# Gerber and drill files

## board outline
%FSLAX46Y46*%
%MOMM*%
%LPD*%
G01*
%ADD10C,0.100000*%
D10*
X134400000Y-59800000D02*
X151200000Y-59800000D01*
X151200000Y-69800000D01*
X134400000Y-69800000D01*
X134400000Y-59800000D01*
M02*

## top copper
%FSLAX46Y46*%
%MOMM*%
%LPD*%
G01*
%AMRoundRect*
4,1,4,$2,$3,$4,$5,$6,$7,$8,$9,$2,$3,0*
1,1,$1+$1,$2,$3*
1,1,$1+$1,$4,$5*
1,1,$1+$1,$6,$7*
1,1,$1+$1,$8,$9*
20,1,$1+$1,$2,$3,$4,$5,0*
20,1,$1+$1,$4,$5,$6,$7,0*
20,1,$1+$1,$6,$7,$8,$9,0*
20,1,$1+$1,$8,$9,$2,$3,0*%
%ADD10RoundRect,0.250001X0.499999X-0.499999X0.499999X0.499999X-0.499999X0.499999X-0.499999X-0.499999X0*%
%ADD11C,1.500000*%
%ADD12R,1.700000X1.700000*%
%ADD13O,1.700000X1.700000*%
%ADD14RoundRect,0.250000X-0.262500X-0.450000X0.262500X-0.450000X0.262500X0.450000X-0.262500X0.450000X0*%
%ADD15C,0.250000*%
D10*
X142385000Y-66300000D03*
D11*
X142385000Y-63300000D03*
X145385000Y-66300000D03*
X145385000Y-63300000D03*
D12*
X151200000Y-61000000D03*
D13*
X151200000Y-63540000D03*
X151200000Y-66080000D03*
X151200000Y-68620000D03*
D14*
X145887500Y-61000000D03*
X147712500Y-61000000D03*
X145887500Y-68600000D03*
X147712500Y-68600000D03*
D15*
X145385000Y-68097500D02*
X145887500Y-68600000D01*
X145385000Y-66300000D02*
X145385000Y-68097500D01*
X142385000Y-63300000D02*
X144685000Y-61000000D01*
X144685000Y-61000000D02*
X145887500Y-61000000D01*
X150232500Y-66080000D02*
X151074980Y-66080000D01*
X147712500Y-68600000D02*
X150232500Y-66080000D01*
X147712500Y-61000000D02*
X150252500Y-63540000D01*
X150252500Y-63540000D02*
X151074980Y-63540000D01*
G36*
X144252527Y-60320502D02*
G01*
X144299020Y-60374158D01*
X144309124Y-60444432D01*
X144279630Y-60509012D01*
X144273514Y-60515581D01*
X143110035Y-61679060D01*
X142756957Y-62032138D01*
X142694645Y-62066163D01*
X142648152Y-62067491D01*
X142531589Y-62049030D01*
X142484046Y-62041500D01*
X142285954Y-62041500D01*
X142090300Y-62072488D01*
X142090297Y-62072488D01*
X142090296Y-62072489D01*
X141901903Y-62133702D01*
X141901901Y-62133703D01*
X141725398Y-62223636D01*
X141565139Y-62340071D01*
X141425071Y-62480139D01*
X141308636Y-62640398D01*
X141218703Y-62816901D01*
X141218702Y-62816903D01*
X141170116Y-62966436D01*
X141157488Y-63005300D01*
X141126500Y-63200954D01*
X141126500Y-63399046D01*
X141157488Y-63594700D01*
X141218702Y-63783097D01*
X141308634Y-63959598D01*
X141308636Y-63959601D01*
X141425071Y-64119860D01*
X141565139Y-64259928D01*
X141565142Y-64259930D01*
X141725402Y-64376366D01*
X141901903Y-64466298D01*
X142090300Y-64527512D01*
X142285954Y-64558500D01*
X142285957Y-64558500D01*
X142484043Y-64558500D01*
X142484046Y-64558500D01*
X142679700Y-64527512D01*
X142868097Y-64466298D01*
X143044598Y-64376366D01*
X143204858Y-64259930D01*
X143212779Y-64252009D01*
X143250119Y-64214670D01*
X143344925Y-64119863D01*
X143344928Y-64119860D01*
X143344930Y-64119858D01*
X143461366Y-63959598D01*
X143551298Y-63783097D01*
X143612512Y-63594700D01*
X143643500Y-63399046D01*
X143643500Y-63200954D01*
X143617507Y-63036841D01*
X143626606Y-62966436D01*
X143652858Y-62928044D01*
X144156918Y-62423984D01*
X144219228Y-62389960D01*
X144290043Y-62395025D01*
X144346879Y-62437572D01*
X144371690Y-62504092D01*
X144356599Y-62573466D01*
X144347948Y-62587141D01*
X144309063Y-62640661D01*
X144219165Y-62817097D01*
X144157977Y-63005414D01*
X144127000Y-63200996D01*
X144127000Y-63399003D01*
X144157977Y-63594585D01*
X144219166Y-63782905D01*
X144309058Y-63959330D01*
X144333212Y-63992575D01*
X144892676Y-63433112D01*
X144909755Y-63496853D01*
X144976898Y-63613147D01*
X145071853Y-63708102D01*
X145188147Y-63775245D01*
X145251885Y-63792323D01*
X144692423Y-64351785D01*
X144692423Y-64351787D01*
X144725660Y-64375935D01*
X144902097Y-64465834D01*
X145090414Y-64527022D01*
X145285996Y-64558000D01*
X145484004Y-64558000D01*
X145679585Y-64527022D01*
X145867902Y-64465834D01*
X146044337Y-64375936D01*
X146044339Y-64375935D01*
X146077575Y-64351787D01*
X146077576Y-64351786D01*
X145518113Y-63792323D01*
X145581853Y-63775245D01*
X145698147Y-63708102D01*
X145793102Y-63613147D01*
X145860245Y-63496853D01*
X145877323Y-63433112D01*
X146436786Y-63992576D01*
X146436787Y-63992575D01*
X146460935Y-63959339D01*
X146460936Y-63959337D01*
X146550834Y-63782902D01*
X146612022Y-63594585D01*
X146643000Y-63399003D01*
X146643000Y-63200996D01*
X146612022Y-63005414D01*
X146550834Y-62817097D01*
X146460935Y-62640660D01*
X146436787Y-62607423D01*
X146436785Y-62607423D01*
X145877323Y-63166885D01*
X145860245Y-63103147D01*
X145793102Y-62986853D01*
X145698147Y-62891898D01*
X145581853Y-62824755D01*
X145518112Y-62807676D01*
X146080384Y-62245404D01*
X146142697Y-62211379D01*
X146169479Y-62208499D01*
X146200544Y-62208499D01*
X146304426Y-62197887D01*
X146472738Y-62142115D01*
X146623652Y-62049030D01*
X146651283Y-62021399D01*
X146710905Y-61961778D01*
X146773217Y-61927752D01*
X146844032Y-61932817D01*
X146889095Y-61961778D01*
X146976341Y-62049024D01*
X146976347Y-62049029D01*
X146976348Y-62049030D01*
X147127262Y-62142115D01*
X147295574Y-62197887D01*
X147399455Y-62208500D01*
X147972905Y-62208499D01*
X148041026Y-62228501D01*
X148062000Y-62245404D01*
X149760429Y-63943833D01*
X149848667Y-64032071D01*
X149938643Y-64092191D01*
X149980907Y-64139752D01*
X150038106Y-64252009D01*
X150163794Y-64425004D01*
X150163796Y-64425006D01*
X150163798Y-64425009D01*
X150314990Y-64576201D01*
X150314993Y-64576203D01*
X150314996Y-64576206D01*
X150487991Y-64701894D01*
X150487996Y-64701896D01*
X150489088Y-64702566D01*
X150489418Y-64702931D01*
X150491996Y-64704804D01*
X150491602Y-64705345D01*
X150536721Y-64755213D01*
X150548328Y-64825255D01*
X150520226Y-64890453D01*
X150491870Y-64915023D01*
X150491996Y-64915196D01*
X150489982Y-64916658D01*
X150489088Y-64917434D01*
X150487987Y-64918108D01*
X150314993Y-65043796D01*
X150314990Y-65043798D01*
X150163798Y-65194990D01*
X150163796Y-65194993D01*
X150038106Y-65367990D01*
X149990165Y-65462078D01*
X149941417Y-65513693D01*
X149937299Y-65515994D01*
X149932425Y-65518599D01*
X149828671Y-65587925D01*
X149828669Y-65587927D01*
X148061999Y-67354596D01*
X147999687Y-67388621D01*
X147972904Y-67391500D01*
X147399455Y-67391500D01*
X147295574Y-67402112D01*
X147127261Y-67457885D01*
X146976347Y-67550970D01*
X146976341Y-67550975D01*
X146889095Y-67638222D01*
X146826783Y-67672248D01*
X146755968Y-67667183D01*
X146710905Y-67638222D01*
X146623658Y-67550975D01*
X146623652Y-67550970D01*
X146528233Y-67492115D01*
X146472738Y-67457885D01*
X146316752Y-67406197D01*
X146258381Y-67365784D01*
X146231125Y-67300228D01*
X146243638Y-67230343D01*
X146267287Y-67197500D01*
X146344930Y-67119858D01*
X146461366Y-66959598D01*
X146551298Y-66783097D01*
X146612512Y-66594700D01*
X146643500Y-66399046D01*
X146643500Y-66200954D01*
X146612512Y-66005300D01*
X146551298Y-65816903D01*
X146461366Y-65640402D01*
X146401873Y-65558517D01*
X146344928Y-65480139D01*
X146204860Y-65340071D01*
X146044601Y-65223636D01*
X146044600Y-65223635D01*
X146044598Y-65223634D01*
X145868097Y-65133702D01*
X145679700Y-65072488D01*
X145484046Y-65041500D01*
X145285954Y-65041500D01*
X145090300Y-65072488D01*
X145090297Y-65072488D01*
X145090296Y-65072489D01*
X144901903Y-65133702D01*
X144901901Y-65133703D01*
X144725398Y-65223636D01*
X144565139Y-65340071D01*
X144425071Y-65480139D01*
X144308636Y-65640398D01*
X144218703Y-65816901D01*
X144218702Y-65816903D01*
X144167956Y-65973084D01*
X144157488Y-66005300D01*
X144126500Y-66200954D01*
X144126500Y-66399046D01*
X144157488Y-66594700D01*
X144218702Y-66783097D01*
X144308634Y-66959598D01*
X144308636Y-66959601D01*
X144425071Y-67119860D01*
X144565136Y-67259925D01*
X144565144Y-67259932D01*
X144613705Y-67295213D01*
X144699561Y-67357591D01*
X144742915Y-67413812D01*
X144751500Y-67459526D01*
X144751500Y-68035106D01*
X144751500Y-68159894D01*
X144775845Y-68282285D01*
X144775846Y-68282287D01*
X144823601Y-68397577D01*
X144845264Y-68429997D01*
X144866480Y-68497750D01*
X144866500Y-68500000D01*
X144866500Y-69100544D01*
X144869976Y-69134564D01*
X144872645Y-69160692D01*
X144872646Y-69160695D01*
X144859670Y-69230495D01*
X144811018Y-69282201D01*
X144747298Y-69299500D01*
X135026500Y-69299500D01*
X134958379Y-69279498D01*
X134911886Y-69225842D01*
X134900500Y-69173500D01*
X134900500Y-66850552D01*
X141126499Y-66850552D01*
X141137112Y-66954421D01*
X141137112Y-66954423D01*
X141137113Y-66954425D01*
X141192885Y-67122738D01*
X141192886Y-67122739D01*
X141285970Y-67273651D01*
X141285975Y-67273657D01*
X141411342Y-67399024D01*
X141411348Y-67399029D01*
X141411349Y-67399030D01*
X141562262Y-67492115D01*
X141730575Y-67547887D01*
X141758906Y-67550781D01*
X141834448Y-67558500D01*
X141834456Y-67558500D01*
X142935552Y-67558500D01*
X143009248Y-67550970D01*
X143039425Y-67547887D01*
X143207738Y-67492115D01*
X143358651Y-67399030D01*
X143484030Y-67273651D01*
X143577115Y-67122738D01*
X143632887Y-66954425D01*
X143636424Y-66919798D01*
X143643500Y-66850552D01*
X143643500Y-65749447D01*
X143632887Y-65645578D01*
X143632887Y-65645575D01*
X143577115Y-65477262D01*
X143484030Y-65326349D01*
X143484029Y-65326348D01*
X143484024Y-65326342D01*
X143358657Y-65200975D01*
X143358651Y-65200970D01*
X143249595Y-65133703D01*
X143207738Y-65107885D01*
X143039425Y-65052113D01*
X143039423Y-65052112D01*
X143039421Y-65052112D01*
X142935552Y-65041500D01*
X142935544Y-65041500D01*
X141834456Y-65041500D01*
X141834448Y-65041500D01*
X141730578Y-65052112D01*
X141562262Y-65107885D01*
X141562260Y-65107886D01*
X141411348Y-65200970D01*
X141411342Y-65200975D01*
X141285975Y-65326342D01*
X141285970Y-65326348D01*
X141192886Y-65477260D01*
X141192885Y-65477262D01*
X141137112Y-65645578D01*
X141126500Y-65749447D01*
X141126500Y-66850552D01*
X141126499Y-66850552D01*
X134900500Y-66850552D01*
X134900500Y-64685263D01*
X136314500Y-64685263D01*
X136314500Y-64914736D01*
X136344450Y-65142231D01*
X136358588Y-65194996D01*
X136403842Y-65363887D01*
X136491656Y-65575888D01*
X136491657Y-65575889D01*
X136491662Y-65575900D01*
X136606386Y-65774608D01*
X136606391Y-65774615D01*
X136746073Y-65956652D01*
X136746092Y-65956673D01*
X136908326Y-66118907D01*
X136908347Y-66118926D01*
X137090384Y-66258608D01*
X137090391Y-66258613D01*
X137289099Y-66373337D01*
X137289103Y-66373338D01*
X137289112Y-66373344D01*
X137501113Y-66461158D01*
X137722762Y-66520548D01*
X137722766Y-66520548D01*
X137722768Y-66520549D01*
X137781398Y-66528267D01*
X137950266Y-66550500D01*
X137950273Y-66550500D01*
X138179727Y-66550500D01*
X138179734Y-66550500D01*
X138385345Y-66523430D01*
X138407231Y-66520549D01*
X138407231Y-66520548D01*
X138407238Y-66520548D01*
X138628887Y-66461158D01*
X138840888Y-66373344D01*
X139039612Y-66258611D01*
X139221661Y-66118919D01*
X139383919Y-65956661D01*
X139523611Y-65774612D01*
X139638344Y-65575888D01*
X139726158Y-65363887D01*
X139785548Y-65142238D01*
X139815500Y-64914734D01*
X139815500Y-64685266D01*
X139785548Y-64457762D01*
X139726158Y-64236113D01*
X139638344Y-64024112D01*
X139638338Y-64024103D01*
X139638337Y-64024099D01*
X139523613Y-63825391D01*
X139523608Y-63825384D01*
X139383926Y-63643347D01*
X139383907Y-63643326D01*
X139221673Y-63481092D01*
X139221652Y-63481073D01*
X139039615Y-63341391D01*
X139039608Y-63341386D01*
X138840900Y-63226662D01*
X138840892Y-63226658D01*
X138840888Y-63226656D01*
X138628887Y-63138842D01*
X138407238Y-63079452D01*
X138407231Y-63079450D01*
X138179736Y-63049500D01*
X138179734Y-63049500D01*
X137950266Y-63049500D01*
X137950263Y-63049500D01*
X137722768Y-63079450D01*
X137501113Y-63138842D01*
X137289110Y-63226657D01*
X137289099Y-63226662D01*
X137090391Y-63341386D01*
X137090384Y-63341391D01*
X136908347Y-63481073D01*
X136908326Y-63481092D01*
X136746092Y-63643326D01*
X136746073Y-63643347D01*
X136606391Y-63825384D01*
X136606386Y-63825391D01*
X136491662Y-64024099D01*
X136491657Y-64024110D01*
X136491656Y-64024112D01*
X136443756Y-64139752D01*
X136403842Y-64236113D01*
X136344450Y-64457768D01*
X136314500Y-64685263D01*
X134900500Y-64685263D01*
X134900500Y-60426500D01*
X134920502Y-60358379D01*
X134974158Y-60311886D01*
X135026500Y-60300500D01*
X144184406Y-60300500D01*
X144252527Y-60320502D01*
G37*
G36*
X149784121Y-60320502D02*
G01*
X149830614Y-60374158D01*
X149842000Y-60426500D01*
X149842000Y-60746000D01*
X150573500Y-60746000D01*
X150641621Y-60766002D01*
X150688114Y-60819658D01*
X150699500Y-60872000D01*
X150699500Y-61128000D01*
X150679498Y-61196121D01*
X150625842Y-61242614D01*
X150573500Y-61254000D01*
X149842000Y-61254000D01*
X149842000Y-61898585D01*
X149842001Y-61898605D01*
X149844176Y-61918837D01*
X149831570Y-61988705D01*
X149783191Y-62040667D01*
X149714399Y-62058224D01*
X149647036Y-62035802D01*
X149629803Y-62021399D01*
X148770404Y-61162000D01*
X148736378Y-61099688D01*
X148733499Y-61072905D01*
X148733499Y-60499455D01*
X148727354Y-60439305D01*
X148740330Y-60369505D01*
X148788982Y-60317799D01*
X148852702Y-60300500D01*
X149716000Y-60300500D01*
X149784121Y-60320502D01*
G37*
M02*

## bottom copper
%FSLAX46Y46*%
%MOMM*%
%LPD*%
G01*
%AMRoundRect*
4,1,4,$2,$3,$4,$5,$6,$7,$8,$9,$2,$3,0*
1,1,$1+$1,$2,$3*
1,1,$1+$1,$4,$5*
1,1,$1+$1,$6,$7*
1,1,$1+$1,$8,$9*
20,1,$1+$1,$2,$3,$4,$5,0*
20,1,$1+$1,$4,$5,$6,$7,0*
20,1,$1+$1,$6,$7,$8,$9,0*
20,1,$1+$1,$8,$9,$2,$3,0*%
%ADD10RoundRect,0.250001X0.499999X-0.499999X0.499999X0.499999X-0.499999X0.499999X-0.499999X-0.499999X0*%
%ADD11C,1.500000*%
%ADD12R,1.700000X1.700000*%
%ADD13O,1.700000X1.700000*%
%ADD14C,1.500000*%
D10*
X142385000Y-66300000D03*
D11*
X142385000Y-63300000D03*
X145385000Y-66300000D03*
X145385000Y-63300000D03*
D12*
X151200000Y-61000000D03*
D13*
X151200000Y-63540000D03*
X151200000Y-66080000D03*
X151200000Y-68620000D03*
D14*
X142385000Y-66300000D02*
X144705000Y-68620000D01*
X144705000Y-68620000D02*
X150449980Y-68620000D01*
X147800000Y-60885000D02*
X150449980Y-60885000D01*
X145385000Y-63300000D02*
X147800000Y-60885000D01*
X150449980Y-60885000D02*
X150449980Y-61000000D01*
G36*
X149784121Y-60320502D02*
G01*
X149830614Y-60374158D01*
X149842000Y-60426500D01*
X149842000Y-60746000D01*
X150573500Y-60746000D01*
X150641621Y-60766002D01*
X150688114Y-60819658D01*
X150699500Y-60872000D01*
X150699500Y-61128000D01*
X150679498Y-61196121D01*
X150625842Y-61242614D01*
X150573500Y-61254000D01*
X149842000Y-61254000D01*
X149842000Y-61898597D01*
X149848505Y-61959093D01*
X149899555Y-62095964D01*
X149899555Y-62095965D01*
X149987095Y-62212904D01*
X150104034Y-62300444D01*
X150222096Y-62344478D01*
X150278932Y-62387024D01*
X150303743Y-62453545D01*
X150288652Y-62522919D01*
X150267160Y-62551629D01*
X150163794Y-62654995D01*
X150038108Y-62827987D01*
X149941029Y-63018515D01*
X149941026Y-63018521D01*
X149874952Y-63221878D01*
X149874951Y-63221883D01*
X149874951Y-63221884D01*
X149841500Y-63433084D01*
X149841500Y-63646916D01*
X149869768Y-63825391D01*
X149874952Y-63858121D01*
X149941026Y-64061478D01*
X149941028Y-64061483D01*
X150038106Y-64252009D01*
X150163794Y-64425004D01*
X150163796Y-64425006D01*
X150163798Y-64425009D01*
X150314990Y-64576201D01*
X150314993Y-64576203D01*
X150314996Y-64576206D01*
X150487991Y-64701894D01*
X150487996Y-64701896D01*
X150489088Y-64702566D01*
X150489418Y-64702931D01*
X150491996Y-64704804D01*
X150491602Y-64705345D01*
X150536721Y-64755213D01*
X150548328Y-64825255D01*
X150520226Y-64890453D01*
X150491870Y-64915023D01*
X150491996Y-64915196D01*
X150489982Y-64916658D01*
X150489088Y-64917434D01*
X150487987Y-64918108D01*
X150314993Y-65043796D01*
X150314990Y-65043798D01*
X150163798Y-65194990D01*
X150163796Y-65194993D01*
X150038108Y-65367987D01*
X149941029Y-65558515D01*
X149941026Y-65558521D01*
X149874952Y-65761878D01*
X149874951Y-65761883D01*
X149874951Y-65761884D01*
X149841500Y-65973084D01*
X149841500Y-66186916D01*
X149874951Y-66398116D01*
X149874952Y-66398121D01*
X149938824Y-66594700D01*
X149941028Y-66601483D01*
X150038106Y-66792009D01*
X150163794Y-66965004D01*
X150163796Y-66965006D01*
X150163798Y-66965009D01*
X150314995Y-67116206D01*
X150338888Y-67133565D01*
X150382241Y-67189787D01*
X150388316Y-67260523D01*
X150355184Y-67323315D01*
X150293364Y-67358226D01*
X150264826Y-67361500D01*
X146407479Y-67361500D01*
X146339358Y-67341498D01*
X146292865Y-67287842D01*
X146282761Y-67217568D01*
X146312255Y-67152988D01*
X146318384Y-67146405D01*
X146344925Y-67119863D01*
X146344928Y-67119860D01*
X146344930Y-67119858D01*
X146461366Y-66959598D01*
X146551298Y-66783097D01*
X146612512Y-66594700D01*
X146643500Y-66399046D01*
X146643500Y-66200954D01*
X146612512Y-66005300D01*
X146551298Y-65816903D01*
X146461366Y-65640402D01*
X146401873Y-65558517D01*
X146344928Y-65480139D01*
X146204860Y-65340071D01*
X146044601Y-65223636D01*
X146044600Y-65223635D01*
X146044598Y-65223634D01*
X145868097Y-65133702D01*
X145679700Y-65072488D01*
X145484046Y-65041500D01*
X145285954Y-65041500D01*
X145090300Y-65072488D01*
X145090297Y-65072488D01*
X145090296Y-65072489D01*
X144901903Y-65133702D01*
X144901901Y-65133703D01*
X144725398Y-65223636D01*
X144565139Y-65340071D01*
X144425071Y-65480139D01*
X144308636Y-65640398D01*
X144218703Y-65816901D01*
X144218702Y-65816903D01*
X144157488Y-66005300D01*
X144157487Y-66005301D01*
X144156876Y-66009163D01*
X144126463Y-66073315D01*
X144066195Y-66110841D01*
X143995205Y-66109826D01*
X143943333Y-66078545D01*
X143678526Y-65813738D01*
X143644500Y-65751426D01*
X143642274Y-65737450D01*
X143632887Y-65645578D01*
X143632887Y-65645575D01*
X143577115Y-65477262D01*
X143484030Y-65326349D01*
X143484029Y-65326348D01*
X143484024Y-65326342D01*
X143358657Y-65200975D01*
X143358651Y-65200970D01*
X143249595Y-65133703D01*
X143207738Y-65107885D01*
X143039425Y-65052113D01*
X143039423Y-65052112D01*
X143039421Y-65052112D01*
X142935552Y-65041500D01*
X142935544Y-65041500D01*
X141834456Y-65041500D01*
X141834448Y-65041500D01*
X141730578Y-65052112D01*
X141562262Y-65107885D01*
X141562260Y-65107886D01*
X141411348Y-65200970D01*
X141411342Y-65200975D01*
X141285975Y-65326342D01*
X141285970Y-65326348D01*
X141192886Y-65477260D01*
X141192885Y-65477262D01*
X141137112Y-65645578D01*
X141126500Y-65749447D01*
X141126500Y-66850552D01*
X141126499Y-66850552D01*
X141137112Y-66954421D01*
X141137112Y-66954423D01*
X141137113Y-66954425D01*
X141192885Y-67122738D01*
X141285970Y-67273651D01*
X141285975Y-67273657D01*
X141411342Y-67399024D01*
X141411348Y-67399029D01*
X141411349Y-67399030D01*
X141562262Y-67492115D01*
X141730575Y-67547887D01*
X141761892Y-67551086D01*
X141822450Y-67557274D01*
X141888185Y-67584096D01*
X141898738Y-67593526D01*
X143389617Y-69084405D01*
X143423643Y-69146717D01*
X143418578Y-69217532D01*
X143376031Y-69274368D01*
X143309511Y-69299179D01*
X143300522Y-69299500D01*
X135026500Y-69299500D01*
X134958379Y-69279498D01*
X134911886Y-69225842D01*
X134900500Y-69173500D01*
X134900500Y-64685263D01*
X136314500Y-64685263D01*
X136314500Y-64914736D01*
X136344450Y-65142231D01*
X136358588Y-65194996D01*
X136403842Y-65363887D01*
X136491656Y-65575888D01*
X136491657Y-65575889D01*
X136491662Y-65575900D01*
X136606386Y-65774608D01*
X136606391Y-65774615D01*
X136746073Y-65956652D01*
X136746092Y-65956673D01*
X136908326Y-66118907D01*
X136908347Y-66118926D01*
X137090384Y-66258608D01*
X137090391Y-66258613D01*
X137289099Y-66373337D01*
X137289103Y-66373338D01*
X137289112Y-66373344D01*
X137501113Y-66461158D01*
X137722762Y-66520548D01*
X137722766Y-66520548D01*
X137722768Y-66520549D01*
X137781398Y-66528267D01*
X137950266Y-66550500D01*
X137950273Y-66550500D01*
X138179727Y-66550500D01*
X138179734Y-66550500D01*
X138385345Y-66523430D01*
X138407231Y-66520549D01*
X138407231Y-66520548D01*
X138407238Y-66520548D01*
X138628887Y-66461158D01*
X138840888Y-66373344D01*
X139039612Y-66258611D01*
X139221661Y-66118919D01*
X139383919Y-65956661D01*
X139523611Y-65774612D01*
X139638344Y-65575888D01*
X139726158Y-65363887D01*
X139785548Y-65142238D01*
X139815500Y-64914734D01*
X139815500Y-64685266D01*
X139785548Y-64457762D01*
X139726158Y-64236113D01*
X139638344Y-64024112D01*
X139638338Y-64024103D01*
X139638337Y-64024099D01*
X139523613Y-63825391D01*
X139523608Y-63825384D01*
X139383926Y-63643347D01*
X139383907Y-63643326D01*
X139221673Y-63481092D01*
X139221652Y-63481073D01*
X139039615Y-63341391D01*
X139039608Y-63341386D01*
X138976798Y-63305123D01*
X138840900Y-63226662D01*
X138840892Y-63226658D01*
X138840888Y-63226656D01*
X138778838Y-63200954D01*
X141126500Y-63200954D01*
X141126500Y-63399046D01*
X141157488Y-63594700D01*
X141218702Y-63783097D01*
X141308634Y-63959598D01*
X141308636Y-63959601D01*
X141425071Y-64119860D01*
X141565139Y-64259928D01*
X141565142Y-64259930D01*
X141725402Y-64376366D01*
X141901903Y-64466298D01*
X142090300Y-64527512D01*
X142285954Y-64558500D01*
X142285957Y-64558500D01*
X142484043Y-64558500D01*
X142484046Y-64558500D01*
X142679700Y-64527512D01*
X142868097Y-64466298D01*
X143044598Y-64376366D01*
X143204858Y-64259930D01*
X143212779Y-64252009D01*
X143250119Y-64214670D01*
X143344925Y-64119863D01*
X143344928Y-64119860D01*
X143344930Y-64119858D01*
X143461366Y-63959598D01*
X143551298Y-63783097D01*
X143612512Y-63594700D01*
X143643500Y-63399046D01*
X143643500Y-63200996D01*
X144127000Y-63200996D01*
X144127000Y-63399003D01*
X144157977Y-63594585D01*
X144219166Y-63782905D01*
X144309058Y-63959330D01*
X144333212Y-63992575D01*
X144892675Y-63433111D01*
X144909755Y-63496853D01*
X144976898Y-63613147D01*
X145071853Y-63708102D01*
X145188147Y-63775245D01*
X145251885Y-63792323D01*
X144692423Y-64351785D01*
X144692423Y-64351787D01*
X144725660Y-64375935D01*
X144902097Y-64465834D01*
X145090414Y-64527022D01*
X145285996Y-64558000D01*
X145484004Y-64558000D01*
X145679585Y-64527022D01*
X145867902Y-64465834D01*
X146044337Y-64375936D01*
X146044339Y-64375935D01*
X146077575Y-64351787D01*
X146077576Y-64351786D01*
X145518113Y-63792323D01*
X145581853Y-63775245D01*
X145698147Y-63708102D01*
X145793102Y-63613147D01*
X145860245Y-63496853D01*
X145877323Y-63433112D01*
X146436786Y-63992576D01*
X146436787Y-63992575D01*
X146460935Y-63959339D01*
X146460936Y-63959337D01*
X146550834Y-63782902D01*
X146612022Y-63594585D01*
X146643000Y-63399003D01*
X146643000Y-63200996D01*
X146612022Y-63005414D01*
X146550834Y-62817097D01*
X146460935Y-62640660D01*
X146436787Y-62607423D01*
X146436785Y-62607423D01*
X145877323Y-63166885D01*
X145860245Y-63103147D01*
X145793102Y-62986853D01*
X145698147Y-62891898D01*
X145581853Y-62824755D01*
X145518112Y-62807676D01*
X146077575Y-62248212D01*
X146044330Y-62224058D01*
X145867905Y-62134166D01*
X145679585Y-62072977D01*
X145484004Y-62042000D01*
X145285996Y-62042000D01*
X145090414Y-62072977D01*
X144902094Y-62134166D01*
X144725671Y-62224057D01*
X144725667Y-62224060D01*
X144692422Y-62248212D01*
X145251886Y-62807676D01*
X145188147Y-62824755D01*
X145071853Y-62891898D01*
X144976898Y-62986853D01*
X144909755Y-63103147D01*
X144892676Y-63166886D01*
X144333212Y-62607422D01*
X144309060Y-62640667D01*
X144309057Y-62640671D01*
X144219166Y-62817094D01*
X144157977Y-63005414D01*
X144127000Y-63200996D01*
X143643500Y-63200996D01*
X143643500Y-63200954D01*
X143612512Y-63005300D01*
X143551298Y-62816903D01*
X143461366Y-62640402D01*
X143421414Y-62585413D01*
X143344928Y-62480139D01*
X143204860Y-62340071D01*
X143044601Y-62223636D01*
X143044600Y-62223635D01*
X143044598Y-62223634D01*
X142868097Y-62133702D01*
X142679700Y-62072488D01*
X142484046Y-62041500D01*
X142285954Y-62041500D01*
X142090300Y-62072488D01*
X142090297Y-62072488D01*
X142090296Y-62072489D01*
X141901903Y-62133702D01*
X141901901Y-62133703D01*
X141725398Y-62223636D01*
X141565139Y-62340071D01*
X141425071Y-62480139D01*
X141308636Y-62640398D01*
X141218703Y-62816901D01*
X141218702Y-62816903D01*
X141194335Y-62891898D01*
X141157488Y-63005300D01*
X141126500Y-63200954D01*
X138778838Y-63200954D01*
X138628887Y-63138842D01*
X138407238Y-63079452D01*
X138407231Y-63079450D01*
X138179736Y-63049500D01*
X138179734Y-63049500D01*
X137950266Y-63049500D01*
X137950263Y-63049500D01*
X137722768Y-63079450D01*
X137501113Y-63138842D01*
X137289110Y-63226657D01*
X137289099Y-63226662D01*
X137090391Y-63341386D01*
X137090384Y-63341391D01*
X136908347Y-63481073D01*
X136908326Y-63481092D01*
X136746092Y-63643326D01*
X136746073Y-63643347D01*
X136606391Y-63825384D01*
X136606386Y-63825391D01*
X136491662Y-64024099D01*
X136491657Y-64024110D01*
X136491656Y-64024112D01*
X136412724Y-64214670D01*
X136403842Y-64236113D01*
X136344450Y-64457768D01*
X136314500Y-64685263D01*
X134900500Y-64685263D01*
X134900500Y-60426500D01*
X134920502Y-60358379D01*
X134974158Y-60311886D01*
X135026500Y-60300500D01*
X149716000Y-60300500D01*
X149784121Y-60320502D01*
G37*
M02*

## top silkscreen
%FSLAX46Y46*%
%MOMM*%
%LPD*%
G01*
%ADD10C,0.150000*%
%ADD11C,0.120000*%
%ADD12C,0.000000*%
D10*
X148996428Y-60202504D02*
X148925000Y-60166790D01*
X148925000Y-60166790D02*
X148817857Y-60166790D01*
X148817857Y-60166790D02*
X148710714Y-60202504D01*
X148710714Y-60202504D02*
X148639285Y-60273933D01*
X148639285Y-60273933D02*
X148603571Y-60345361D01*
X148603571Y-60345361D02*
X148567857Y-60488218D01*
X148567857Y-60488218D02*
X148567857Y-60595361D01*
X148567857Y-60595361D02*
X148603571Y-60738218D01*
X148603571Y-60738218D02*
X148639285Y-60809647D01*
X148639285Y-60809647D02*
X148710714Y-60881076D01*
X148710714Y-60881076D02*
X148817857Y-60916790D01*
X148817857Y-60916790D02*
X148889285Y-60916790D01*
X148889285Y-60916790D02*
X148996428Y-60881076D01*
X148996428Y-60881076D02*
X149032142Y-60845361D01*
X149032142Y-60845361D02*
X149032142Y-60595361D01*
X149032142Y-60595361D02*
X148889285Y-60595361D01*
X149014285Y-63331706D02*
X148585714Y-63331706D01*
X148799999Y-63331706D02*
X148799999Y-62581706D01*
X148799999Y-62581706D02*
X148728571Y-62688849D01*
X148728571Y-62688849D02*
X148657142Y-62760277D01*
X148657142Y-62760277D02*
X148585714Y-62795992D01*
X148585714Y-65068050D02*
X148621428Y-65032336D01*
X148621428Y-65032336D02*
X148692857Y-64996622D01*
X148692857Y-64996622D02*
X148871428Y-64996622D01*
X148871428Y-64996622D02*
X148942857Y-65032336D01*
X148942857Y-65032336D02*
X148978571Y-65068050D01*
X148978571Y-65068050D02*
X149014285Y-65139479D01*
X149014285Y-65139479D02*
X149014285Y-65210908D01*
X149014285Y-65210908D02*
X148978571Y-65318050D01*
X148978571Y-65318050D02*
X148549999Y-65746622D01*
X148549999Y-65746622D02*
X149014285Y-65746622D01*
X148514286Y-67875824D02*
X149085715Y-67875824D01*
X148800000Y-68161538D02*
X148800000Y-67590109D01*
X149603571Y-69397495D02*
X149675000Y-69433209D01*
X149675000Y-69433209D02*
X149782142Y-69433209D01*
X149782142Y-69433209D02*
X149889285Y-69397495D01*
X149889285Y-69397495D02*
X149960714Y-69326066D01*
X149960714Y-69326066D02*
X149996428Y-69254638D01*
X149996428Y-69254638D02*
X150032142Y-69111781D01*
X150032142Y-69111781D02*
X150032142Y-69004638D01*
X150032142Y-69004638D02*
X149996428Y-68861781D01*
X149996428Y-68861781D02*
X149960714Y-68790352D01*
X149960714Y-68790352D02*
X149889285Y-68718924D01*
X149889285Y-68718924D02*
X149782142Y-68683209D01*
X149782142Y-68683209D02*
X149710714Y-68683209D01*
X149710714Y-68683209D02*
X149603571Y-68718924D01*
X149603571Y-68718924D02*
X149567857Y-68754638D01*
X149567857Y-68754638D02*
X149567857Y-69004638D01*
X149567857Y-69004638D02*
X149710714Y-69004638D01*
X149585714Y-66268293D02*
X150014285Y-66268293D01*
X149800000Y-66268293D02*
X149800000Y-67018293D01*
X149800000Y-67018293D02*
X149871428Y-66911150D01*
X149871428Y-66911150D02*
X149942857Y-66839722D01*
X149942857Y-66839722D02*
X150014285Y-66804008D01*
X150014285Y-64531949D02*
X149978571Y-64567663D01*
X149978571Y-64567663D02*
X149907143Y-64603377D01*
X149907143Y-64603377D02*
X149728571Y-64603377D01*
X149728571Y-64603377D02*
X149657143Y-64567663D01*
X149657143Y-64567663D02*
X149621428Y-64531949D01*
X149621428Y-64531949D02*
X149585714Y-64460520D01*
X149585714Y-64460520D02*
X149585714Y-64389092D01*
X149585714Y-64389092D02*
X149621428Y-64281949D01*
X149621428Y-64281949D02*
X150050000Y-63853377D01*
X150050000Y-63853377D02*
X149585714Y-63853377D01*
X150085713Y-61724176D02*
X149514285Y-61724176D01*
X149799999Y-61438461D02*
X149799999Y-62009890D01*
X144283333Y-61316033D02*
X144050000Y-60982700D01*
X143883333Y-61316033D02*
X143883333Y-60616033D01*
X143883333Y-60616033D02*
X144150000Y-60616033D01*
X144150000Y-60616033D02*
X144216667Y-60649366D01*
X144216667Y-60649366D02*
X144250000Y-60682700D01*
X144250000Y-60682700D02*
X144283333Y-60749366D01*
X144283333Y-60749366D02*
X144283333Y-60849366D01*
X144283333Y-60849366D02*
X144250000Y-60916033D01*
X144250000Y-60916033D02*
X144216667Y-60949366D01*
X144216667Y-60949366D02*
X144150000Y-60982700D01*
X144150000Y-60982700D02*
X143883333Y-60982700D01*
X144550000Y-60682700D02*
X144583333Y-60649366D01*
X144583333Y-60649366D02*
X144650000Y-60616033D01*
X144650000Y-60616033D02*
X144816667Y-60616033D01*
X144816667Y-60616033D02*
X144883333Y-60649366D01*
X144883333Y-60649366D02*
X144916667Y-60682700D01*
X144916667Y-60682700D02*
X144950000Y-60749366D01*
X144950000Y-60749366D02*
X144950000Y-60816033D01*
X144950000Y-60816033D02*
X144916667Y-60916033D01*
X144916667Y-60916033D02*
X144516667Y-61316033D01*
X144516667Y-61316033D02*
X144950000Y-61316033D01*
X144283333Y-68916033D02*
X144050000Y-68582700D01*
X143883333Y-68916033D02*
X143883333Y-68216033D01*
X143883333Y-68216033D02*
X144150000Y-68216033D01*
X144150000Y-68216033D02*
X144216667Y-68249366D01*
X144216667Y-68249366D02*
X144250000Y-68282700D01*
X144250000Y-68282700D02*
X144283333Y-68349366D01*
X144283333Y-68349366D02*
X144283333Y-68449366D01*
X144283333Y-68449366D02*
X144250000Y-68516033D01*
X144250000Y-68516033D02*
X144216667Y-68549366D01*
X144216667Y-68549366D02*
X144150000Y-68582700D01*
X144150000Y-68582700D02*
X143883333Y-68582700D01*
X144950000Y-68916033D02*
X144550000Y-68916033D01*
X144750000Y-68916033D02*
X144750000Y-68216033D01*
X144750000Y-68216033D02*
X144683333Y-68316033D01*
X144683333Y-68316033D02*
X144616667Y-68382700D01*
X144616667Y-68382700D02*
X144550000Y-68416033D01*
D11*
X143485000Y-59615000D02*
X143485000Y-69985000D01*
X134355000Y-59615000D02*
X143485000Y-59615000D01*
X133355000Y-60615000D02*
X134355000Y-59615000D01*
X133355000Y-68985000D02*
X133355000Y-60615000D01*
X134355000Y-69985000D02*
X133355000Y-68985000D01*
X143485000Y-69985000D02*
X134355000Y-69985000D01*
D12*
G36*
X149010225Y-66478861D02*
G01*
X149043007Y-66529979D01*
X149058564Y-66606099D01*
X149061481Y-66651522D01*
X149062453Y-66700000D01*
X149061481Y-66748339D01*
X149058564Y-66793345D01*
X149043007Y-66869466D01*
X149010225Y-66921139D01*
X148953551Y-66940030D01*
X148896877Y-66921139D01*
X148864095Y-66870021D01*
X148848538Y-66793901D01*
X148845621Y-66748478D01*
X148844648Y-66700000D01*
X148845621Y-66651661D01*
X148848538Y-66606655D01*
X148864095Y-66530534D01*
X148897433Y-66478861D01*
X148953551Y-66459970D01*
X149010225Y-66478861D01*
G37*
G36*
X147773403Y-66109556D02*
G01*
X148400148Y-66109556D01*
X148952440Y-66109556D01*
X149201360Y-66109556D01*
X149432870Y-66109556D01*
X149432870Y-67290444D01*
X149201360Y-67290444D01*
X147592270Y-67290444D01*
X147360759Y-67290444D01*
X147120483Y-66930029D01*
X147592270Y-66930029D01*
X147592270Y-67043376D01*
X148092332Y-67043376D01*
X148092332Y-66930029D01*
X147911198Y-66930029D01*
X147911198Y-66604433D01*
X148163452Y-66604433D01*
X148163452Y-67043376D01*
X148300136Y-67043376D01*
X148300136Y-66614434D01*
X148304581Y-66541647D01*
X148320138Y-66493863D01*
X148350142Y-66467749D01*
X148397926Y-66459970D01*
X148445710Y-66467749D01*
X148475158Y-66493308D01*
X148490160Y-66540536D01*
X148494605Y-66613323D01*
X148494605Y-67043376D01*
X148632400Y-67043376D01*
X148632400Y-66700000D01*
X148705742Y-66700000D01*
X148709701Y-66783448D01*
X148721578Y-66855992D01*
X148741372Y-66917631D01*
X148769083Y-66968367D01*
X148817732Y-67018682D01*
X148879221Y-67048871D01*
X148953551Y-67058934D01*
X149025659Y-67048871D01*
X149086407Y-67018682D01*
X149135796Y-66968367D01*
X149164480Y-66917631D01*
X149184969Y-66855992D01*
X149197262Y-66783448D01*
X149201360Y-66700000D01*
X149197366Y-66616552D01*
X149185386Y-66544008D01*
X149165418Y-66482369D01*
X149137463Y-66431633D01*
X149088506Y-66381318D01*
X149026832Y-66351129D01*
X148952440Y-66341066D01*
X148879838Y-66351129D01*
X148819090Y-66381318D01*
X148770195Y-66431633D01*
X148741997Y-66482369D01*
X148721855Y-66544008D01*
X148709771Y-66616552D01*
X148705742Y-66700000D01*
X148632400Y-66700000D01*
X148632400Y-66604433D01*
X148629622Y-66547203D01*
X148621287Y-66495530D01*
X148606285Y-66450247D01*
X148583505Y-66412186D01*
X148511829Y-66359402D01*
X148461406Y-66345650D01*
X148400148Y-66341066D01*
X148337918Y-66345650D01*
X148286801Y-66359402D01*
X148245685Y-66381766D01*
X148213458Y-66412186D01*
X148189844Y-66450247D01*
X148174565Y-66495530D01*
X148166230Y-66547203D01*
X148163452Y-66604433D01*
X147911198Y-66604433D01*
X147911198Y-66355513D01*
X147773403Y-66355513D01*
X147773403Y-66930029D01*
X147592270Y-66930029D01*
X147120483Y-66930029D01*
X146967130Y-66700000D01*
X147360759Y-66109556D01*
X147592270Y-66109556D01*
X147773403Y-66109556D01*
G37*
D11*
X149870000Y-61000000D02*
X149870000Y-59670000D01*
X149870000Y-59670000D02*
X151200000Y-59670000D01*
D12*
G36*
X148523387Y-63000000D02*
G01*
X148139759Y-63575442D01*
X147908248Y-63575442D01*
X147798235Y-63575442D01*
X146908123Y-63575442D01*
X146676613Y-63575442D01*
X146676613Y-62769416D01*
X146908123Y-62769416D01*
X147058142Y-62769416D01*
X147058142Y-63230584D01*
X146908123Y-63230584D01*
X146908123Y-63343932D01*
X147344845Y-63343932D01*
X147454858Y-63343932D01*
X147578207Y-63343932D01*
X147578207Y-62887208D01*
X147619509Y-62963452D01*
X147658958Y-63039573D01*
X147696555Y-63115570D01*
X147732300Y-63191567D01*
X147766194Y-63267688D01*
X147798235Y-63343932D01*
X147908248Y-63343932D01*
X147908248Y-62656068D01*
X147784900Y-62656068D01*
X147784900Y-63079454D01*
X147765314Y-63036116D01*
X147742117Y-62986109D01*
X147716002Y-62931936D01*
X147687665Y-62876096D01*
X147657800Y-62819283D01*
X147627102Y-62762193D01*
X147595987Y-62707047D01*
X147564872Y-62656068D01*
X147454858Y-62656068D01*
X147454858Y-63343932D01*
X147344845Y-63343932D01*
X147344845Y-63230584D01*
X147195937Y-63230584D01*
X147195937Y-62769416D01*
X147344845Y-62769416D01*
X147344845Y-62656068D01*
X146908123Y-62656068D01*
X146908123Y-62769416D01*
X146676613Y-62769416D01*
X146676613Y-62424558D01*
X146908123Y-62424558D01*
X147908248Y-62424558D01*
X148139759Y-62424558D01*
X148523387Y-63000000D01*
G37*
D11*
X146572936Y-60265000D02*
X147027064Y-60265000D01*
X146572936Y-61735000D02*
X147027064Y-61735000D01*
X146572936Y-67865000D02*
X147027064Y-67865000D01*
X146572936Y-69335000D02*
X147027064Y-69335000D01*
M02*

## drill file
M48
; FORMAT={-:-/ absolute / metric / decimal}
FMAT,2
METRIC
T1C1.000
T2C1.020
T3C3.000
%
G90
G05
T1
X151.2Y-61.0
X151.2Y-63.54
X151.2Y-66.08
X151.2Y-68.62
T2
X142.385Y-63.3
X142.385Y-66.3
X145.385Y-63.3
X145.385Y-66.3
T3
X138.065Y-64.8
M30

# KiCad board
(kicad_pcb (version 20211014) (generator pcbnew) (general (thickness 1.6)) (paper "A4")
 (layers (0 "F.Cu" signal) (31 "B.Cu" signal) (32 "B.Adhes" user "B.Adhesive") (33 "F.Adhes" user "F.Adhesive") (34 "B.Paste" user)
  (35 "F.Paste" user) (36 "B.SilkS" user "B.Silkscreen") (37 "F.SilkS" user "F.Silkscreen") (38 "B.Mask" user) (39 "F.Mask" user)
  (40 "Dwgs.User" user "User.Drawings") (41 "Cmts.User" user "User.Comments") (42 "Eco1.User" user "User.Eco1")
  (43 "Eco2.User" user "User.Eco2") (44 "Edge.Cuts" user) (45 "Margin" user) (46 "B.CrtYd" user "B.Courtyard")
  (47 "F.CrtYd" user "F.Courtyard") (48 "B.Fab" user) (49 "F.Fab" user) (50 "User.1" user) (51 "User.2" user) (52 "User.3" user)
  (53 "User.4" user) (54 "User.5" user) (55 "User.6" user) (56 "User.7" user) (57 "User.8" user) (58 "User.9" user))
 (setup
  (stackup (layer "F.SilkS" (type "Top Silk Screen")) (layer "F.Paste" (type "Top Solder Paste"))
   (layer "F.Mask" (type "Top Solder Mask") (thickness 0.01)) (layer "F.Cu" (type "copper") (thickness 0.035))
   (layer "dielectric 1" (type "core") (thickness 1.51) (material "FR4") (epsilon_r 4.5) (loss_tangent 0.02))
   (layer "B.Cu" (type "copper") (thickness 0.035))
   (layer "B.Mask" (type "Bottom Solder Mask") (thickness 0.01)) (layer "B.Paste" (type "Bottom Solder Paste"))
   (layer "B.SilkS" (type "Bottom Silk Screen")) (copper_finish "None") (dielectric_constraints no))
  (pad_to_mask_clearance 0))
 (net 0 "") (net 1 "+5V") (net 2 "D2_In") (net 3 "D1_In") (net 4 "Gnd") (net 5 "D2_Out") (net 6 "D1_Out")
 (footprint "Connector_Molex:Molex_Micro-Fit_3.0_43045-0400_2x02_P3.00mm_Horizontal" (layer "F.Cu") (at 142.385 66.3 90)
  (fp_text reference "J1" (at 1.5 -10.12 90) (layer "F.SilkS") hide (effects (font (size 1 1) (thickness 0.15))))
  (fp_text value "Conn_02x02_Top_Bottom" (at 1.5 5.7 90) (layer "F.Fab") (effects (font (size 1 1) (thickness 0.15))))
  (fp_line (start 6.685 1.1) (end -3.685 1.1) (layer "F.SilkS") (width 0.12))
  (fp_line (start 6.685 -8.03) (end 6.685 1.1) (layer "F.SilkS") (width 0.12))
  (fp_line (start 5.685 -9.03) (end 6.685 -8.03) (layer "F.SilkS") (width 0.12))
  (fp_line (start -2.685 -9.03) (end 5.685 -9.03) (layer "F.SilkS") (width 0.12))
  (fp_line (start -3.685 -8.03) (end -2.685 -9.03) (layer "F.SilkS") (width 0.12))
  (fp_line (start -3.685 1.1) (end -3.685 -8.03) (layer "F.SilkS") (width 0.12))
  (pad "" np_thru_hole circle locked (at 1.5 -4.32 90) (size 3 3) (drill 3) (layers *.Cu *.Mask))
  (pad "1" thru_hole roundrect locked (at 0 0 90) (size 1.5 1.5) (drill 1.02) (layers *.Cu *.Mask) (roundrect_rratio 0.1666673333)
   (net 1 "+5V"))
  (pad "2" thru_hole circle locked (at 3 0 90) (size 1.5 1.5) (drill 1.02) (layers *.Cu *.Mask) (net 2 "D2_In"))
  (pad "3" thru_hole circle locked (at 0 3 90) (size 1.5 1.5) (drill 1.02) (layers *.Cu *.Mask) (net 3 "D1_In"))
  (pad "4" thru_hole circle locked (at 3 3 90) (size 1.5 1.5) (drill 1.02) (layers *.Cu *.Mask) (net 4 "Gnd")))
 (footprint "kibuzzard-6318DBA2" (layer "F.Cu") (at 148.2 66.7 180)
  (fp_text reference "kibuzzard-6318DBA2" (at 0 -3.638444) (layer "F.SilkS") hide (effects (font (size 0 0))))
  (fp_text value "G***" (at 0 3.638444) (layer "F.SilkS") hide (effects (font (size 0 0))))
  (fp_poly
   (pts (xy -0.862453 0) (xy -0.861481 0.048478) (xy -0.858564 0.093901) (xy -0.843007 0.170021) (xy -0.810225 0.221139)
    (xy -0.753551 0.24003) (xy -0.697433 0.221139) (xy -0.664095 0.169466) (xy -0.648538 0.093345) (xy -0.645621 0.048339) (xy -0.644648 0)
    (xy -0.645621 -0.048478) (xy -0.648538 -0.093901) (xy -0.664095 -0.170021) (xy -0.696877 -0.221139) (xy -0.753551 -0.24003)
    (xy -0.810225 -0.221139) (xy -0.843007 -0.169466) (xy -0.858564 -0.093345) (xy -0.861481 -0.048339) (xy -0.862453 0))
   (layer "F.SilkS") (width 0) (fill solid))
  (fp_poly
   (pts (xy -1.00136 -0.590444) (xy -1.23287 -0.590444) (xy -1.23287 0.590444) (xy -1.00136 0.590444) (xy -0.75244 0.590444)
    (xy -0.75244 0.358934) (xy -0.826832 0.348871) (xy -0.888506 0.318682) (xy -0.937463 0.268367) (xy -0.965418 0.217631)
    (xy -0.985386 0.155992) (xy -0.997366 0.083448) (xy -1.00136 0) (xy -0.997262 -0.083448) (xy -0.984969 -0.155992)
    (xy -0.96448 -0.217631) (xy -0.935796 -0.268367) (xy -0.886407 -0.318682) (xy -0.825659 -0.348871) (xy -0.753551 -0.358934)
    (xy -0.679221 -0.348871) (xy -0.617732 -0.318682) (xy -0.569083 -0.268367) (xy -0.541372 -0.217631) (xy -0.521578 -0.155992)
    (xy -0.509701 -0.083448) (xy -0.505742 0) (xy -0.509771 0.083448) (xy -0.521855 0.155992) (xy -0.541997 0.217631)
    (xy -0.570195 0.268367) (xy -0.61909 0.318682) (xy -0.679838 0.348871) (xy -0.75244 0.358934) (xy -0.75244 0.590444)
    (xy -0.200148 0.590444) (xy -0.200148 0.358934) (xy -0.261406 0.35435) (xy -0.311829 0.340598) (xy -0.383505 0.287814)
    (xy -0.406285 0.249753) (xy -0.421287 0.20447) (xy -0.429622 0.152797) (xy -0.4324 0.095567) (xy -0.4324 -0.343376)
    (xy -0.294605 -0.343376) (xy -0.294605 0.086677) (xy -0.29016 0.159464) (xy -0.275158 0.206692) (xy -0.24571 0.232251)
    (xy -0.197926 0.24003) (xy -0.150142 0.232251) (xy -0.120138 0.206137) (xy -0.104581 0.158353) (xy -0.100136 0.085566)
    (xy -0.100136 -0.343376) (xy 0.036548 -0.343376) (xy 0.036548 0.095567) (xy 0.03377 0.152797) (xy 0.025435 0.20447)
    (xy 0.010156 0.249753) (xy -0.013458 0.287814) (xy -0.045685 0.318234) (xy -0.086801 0.340598) (xy -0.137918 0.35435)
    (xy -0.200148 0.358934) (xy -0.200148 0.590444) (xy 0.426597 0.590444) (xy 0.426597 0.344487) (xy 0.288802 0.344487)
    (xy 0.288802 -0.230029) (xy 0.107668 -0.230029) (xy 0.107668 -0.343376) (xy 0.60773 -0.343376) (xy 0.60773 -0.230029)
    (xy 0.426597 -0.230029) (xy 0.426597 0.344487) (xy 0.426597 0.590444) (xy 0.60773 0.590444) (xy 0.839241 0.590444) (xy 1.23287 0)
    (xy 0.839241 -0.590444) (xy 0.60773 -0.590444) (xy -1.00136 -0.590444))
   (layer "F.SilkS") (width 0) (fill solid)))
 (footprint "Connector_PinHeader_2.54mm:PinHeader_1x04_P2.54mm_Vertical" (layer "F.Cu") (at 151.2 61)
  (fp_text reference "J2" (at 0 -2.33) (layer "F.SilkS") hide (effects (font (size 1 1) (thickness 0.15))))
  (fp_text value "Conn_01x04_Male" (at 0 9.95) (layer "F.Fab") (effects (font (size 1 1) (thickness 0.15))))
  (fp_line (start -1.33 0) (end -1.33 -1.33) (layer "F.SilkS") (width 0.12))
  (fp_line (start -1.33 -1.33) (end 0 -1.33) (layer "F.SilkS") (width 0.12))
  (pad "1" thru_hole rect (at 0 0) (size 1.7 1.7) (drill 1) (layers *.Cu *.Mask) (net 4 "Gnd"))
  (pad "2" thru_hole oval (at 0 2.54) (size 1.7 1.7) (drill 1) (layers *.Cu *.Mask) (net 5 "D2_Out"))
  (pad "3" thru_hole oval (at 0 5.08) (size 1.7 1.7) (drill 1) (layers *.Cu *.Mask) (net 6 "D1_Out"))
  (pad "4" thru_hole oval (at 0 7.62) (size 1.7 1.7) (drill 1) (layers *.Cu *.Mask) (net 1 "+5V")))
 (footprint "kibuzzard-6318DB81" (layer "F.Cu") (at 147.6 63)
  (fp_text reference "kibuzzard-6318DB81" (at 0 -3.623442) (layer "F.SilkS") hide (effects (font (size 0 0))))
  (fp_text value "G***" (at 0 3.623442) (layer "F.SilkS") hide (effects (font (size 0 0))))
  (fp_poly
   (pts (xy -0.691877 -0.575442) (xy -0.923387 -0.575442) (xy -0.923387 0.575442) (xy -0.691877 0.575442) (xy -0.691877 0.343932)
    (xy -0.691877 0.230584) (xy -0.541858 0.230584) (xy -0.541858 -0.230584) (xy -0.691877 -0.230584) (xy -0.691877 -0.343932)
    (xy -0.255155 -0.343932) (xy -0.255155 -0.230584) (xy -0.404063 -0.230584) (xy -0.404063 0.230584) (xy -0.255155 0.230584)
    (xy -0.255155 0.343932) (xy -0.691877 0.343932) (xy -0.691877 0.575442) (xy 0.198235 0.575442) (xy 0.198235 0.343932)
    (xy 0.166194 0.267688) (xy 0.1323 0.191567) (xy 0.096555 0.11557) (xy 0.058958 0.039573) (xy 0.019509 -0.036548)
    (xy -0.021793 -0.112792) (xy -0.021793 0.343932) (xy -0.145142 0.343932) (xy -0.145142 -0.343932) (xy -0.035128 -0.343932)
    (xy -0.004013 -0.292953) (xy 0.027102 -0.237807) (xy 0.0578 -0.180717) (xy 0.087665 -0.123904) (xy 0.116002 -0.068064)
    (xy 0.142117 -0.013891) (xy 0.165314 0.036116) (xy 0.1849 0.079454) (xy 0.1849 -0.343932) (xy 0.308248 -0.343932) (xy 0.308248 0.343932)
    (xy 0.198235 0.343932) (xy 0.198235 0.575442) (xy 0.308248 0.575442) (xy 0.539759 0.575442) (xy 0.923387 0) (xy 0.539759 -0.575442)
    (xy 0.308248 -0.575442) (xy -0.691877 -0.575442))
   (layer "F.SilkS") (width 0) (fill solid)))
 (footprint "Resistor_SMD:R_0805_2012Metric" (layer "F.Cu") (at 146.8 61)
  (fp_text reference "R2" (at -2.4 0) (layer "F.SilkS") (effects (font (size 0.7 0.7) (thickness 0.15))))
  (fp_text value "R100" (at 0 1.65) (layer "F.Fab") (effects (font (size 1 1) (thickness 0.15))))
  (fp_line (start -0.227064 -0.735) (end 0.227064 -0.735) (layer "F.SilkS") (width 0.12))
  (fp_line (start -0.227064 0.735) (end 0.227064 0.735) (layer "F.SilkS") (width 0.12))
  (pad "1" smd roundrect locked (at -0.9125 0) (size 1.025 1.4) (layers "F.Cu" "F.Paste" "F.Mask") (roundrect_rratio 0.243902439)
   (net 2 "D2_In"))
  (pad "2" smd roundrect locked (at 0.9125 0) (size 1.025 1.4) (layers "F.Cu" "F.Paste" "F.Mask") (roundrect_rratio 0.243902439)
   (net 5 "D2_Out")))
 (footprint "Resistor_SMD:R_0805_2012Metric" (layer "F.Cu") (at 146.8 68.6)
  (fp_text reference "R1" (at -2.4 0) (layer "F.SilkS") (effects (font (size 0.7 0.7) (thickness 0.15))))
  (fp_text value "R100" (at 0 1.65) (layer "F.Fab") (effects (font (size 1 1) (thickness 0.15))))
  (fp_line (start -0.227064 -0.735) (end 0.227064 -0.735) (layer "F.SilkS") (width 0.12))
  (fp_line (start -0.227064 0.735) (end 0.227064 0.735) (layer "F.SilkS") (width 0.12))
  (pad "1" smd roundrect locked (at -0.9125 0) (size 1.025 1.4) (layers "F.Cu" "F.Paste" "F.Mask") (roundrect_rratio 0.243902439)
   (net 3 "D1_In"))
  (pad "2" smd roundrect locked (at 0.9125 0) (size 1.025 1.4) (layers "F.Cu" "F.Paste" "F.Mask") (roundrect_rratio 0.243902439)
   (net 6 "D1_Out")))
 (gr_rect (start 134.4 59.8) (end 151.2 69.8) (layer "Edge.Cuts") (width 0.1) (fill none))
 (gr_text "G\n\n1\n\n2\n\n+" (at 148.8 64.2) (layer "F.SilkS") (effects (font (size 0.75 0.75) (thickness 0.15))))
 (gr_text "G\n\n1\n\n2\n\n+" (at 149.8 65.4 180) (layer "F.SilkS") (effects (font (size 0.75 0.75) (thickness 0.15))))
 (segment (start 142.385 66.3) (end 144.705 68.62) (width 1.5) (layer "B.Cu") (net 1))
 (segment (start 144.705 68.62) (end 150.44998 68.62) (width 1.5) (layer "B.Cu") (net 1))
 (segment (start 145.385 68.0975) (end 145.8875 68.6) (width 0.25) (layer "F.Cu") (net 3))
 (segment (start 145.385 66.3) (end 145.385 68.0975) (width 0.25) (layer "F.Cu") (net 3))
 (segment (start 142.385 63.3) (end 144.685 61) (width 0.25) (layer "F.Cu") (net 2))
 (segment (start 144.685 61) (end 145.8875 61) (width 0.25) (layer "F.Cu") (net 2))
 (segment (start 147.8 60.885) (end 150.44998 60.885) (width 1.5) (layer "B.Cu") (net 4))
 (segment (start 145.385 63.3) (end 147.8 60.885) (width 1.5) (layer "B.Cu") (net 4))
 (segment (start 150.44998 60.885) (end 150.44998 61) (width 1.5) (layer "B.Cu") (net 4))
 (segment (start 150.2325 66.08) (end 151.07498 66.08) (width 0.25) (layer "F.Cu") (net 6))
 (segment (start 147.7125 68.6) (end 150.2325 66.08) (width 0.25) (layer "F.Cu") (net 6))
 (segment (start 147.7125 61) (end 150.2525 63.54) (width 0.25) (layer "F.Cu") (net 5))
 (segment (start 150.2525 63.54) (end 151.07498 63.54) (width 0.25) (layer "F.Cu") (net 5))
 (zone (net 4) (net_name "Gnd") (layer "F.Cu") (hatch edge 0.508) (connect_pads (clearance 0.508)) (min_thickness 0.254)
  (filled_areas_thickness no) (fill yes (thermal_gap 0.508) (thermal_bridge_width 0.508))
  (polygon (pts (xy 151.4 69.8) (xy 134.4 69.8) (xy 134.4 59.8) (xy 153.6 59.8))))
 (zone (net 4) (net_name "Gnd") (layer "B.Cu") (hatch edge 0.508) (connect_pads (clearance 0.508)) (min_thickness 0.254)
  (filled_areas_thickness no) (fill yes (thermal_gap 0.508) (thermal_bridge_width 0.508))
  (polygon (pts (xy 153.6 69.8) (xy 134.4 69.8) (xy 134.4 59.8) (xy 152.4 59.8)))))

